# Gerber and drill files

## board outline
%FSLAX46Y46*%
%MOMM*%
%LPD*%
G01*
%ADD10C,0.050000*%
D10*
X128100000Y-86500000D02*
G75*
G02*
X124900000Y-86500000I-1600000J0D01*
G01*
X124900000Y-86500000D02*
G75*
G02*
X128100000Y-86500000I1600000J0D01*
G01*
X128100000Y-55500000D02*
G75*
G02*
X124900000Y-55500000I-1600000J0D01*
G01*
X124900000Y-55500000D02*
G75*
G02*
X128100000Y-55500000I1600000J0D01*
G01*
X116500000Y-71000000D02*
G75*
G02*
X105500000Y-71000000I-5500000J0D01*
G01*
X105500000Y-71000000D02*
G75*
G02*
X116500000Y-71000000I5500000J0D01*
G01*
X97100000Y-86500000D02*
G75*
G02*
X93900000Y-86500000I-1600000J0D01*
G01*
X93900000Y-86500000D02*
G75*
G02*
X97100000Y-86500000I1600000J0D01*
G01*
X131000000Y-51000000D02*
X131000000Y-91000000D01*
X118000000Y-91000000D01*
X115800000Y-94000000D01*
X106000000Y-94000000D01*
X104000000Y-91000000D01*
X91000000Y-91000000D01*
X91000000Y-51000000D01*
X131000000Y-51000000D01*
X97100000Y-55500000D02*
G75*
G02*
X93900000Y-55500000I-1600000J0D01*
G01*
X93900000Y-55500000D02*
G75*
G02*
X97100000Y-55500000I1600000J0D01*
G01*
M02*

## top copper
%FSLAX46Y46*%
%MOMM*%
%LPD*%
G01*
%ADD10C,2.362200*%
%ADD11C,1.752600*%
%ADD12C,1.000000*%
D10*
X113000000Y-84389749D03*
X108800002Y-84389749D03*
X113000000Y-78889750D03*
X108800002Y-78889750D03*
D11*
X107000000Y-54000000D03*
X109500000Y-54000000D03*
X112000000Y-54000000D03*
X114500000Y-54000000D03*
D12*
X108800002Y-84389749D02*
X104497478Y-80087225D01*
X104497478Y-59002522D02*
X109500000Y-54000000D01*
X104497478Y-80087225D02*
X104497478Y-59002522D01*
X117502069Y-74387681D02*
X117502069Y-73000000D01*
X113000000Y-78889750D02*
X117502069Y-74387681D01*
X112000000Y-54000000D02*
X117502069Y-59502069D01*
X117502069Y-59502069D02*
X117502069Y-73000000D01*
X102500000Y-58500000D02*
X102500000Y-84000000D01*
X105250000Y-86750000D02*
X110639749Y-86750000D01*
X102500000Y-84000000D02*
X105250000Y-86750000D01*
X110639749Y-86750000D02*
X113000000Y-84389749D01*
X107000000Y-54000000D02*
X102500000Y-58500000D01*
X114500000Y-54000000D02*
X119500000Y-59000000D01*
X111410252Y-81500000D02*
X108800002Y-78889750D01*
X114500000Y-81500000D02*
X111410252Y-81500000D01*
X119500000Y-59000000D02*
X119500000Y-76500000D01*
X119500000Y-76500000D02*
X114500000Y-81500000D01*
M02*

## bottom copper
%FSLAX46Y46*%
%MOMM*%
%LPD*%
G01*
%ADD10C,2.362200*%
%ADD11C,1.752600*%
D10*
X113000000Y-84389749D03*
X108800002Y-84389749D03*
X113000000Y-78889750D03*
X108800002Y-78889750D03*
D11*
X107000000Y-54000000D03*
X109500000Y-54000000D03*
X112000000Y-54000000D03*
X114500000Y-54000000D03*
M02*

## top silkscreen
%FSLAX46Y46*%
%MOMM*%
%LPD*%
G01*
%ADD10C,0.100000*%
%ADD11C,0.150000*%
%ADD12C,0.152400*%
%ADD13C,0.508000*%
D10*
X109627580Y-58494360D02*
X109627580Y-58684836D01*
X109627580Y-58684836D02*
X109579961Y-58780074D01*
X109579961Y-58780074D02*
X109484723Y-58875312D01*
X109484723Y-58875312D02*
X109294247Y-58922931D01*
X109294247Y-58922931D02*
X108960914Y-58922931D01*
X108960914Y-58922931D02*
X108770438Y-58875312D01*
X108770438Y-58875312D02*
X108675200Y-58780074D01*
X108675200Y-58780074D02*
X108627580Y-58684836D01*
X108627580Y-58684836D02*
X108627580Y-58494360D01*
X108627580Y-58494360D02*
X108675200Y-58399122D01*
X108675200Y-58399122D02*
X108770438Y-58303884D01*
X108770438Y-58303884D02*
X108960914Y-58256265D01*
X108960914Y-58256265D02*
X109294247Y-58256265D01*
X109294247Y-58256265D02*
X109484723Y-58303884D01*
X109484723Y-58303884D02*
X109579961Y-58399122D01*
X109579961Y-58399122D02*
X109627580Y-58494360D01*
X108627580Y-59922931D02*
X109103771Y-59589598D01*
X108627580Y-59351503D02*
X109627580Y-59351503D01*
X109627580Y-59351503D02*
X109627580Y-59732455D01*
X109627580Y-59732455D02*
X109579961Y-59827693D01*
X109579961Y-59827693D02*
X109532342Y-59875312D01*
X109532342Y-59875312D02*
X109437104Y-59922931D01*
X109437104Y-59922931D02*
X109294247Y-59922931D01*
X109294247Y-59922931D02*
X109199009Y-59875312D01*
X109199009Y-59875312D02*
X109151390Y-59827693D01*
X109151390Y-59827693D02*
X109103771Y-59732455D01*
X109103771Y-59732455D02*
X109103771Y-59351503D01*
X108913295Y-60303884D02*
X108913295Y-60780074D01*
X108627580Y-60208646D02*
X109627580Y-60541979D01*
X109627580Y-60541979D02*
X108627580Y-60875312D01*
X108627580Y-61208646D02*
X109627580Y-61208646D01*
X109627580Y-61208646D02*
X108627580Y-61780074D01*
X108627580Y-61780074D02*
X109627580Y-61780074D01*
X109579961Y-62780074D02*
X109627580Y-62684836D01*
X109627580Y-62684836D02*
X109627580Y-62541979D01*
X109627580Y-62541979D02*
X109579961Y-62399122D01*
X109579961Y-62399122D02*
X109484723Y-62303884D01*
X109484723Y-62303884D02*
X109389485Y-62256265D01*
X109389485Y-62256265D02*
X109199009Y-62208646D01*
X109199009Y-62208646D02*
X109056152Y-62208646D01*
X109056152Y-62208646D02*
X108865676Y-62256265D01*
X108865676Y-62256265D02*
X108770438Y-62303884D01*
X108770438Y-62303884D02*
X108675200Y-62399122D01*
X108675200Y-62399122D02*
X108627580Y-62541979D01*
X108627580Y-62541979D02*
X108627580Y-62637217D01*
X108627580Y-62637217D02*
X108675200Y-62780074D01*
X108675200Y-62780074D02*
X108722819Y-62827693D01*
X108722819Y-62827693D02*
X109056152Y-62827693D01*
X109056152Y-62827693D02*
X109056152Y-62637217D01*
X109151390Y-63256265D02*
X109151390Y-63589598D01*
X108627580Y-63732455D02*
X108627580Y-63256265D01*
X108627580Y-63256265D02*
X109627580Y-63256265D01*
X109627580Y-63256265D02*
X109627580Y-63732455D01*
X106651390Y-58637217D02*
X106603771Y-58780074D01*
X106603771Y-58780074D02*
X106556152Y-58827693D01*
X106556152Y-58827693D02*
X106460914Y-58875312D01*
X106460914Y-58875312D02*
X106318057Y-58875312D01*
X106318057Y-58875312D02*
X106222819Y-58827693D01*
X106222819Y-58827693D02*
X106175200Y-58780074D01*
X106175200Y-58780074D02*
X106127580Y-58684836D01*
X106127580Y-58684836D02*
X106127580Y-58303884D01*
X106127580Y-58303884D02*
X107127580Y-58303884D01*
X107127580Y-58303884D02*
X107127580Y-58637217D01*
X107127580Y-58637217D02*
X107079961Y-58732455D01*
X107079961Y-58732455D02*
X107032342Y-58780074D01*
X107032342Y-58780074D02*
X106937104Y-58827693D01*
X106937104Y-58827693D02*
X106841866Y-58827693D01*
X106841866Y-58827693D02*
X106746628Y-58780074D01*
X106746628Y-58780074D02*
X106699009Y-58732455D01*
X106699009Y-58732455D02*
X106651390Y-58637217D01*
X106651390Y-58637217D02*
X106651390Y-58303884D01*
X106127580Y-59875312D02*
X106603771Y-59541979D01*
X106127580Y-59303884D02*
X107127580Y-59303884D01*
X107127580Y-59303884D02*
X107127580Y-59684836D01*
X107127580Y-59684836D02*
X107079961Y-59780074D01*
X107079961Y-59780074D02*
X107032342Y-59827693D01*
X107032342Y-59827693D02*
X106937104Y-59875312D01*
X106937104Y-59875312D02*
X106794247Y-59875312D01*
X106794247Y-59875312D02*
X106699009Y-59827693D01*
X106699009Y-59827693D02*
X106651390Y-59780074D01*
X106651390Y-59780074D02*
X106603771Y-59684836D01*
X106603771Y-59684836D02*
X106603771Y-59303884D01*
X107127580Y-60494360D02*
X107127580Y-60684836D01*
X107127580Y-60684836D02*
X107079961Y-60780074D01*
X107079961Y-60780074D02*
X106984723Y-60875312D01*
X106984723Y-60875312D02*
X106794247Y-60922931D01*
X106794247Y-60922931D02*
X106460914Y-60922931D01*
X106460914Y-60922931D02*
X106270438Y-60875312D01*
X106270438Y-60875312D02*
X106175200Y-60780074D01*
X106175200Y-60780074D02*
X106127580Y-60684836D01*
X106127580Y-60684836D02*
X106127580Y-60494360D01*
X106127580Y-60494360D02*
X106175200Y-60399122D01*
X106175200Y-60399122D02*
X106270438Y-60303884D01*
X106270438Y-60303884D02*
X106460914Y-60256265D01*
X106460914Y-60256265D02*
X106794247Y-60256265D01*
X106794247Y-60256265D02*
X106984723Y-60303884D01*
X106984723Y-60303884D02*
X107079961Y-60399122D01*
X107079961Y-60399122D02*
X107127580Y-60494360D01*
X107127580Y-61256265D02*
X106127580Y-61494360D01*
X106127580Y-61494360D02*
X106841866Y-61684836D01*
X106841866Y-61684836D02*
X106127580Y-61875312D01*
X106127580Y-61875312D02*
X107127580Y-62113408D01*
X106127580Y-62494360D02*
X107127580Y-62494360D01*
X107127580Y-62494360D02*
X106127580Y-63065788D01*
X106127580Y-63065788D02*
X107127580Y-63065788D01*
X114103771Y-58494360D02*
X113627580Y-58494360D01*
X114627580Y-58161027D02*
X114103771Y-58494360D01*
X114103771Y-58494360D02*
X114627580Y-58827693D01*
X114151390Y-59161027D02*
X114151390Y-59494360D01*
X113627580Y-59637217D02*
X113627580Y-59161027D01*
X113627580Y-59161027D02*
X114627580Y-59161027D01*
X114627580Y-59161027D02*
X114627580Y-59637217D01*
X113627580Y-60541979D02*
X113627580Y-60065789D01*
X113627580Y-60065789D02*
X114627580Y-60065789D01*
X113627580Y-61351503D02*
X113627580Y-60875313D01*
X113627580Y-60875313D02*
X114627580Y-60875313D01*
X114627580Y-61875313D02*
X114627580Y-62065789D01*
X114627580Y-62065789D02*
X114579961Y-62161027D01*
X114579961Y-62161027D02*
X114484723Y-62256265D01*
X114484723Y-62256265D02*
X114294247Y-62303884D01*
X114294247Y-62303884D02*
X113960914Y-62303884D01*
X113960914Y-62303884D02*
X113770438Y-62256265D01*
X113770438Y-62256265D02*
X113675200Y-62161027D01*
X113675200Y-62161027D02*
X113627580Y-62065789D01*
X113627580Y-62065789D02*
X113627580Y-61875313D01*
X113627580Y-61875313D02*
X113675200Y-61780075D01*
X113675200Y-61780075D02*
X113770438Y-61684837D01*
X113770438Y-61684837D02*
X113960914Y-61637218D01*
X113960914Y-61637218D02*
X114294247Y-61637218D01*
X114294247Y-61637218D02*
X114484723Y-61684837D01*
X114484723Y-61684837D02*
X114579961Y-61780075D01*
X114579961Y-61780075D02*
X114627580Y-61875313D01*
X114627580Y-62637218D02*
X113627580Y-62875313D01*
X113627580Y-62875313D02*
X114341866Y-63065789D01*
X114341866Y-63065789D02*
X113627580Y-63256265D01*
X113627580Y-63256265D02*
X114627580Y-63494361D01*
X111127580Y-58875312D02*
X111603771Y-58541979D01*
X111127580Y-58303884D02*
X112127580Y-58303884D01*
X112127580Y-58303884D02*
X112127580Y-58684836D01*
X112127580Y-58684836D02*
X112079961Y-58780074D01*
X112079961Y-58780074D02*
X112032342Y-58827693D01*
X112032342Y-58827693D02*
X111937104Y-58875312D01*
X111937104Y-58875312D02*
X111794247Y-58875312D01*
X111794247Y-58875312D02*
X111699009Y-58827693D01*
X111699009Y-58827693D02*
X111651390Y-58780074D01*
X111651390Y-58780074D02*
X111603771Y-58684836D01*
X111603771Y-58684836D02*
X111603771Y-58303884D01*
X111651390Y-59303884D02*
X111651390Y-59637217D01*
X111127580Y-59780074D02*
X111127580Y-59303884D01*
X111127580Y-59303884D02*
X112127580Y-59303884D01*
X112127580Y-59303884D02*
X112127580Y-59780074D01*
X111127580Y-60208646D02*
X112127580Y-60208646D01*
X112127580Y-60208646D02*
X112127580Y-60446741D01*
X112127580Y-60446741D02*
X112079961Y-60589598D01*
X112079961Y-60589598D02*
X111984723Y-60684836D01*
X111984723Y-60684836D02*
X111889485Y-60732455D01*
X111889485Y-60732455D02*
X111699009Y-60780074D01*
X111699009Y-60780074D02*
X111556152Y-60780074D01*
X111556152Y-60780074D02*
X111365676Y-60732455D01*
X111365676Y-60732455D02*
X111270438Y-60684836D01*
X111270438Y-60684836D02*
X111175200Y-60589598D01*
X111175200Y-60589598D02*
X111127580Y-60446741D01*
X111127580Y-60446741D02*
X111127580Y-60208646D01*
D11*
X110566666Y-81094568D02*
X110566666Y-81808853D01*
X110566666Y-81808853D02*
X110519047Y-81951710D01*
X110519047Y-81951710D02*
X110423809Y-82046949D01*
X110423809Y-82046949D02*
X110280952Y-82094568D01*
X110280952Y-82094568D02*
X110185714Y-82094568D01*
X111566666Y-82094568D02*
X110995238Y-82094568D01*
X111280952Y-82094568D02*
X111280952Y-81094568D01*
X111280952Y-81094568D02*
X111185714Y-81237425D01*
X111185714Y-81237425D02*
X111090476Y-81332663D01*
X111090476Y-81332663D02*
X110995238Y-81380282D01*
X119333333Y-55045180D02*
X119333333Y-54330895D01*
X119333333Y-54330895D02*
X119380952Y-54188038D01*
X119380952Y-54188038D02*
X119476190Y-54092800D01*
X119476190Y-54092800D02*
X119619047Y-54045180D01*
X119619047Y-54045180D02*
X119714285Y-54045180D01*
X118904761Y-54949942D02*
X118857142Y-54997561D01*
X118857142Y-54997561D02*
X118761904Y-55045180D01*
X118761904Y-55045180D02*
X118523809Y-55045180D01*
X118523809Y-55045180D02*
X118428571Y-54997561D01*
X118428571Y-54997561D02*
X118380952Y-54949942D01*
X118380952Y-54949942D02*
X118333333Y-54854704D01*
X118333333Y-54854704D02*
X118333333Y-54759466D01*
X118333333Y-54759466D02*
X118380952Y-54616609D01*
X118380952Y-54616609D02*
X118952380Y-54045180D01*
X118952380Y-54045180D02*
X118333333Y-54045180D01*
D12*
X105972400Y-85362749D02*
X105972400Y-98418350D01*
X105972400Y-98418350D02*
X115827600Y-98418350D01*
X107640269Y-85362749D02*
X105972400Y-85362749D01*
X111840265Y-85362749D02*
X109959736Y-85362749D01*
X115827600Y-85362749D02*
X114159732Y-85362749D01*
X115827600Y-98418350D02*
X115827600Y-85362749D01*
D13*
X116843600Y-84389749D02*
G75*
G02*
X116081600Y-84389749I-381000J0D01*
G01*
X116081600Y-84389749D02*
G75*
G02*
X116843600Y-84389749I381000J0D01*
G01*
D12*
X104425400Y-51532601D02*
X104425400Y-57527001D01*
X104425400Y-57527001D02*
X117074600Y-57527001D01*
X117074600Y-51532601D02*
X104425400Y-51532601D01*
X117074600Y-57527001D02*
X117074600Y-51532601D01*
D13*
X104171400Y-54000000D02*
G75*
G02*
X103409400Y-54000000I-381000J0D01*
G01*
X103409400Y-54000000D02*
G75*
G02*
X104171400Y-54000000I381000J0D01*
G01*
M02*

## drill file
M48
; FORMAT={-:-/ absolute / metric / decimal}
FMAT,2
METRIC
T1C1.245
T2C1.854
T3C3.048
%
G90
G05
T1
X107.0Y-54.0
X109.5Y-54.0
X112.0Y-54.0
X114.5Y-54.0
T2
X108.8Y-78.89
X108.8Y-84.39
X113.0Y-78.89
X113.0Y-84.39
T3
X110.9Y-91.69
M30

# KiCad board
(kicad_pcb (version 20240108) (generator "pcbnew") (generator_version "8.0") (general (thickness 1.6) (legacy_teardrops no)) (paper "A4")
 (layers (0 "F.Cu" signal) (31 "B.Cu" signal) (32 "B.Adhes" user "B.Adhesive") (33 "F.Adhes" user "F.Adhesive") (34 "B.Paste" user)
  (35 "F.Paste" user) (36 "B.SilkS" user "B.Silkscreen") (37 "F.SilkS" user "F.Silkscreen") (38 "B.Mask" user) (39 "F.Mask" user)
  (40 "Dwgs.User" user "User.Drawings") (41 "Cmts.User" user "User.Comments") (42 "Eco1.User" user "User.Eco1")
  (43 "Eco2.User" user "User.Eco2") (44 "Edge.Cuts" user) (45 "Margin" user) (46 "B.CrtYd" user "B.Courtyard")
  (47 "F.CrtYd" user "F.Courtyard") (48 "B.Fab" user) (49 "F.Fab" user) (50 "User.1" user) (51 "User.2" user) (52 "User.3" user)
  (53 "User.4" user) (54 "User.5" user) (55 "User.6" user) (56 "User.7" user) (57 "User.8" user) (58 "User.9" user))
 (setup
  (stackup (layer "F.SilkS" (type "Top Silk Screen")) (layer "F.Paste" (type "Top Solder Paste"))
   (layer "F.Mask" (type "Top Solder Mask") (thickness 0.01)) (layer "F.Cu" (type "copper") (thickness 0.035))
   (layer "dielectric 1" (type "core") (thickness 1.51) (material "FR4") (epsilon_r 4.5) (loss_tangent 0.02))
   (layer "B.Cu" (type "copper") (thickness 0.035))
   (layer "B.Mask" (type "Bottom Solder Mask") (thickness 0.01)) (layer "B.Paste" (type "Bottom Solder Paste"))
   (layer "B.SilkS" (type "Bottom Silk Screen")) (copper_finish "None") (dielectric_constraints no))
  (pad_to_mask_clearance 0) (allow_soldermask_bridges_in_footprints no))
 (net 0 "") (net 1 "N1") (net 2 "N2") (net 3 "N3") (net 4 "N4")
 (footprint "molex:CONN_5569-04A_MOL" (layer "F.Cu") (at 113 84.389749)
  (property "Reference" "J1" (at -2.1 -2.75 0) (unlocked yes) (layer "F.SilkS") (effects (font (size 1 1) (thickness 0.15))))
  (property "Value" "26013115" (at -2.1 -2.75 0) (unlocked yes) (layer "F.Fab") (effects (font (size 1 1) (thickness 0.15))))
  (fp_line (start -7.0276 0.973) (end -7.0276 14.028601) (stroke (width 0.1524) (type solid)) (layer "F.SilkS"))
  (fp_line (start -7.0276 14.028601) (end 2.8276 14.028601) (stroke (width 0.1524) (type solid)) (layer "F.SilkS"))
  (fp_line (start -5.359731 0.973) (end -7.0276 0.973) (stroke (width 0.1524) (type solid)) (layer "F.SilkS"))
  (fp_line (start -1.159735 0.973) (end -3.040264 0.973) (stroke (width 0.1524) (type solid)) (layer "F.SilkS"))
  (fp_line (start 2.8276 0.973) (end 1.159732 0.973) (stroke (width 0.1524) (type solid)) (layer "F.SilkS"))
  (fp_line (start 2.8276 14.028601) (end 2.8276 0.973) (stroke (width 0.1524) (type solid)) (layer "F.SilkS"))
  (fp_circle (center 3.4626 0) (end 3.8436 0) (stroke (width 0.508) (type solid)) (fill none) (layer "F.SilkS"))
  (pad "" np_thru_hole circle (at -2.1 7.300001) (size 3.048 3.048) (drill 3.048) (layers))
  (pad "1" thru_hole circle (at 0 0) (size 2.3622 2.3622) (drill 1.8542) (layers "*.Cu" "*.Mask") (remove_unused_layers no) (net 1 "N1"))
  (pad "2" thru_hole circle (at -4.199998 0) (size 2.3622 2.3622) (drill 1.8542) (layers "*.Cu" "*.Mask") (remove_unused_layers no)
   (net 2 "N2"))
  (pad "3" thru_hole circle (at 0 -5.499999) (size 2.3622 2.3622) (drill 1.8542) (layers "*.Cu" "*.Mask") (remove_unused_layers no)
   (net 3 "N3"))
  (pad "4" thru_hole circle (at -4.199998 -5.499999) (size 2.3622 2.3622) (drill 1.8542) (layers "*.Cu" "*.Mask") (remove_unused_layers no)
   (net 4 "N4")))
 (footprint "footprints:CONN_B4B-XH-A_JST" (layer "F.Cu") (at 107 54 180)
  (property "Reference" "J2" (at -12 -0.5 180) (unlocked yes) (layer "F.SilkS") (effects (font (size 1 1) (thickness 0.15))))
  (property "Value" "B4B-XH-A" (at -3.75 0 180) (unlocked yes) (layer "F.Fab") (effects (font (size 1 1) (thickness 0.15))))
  (fp_line (start 2.5746 2.467399) (end 2.5746 -3.527001) (stroke (width 0.1524) (type solid)) (layer "F.SilkS"))
  (fp_line (start 2.5746 -3.527001) (end -10.0746 -3.527001) (stroke (width 0.1524) (type solid)) (layer "F.SilkS"))
  (fp_line (start -10.0746 2.467399) (end 2.5746 2.467399) (stroke (width 0.1524) (type solid)) (layer "F.SilkS"))
  (fp_line (start -10.0746 -3.527001) (end -10.0746 2.467399) (stroke (width 0.1524) (type solid)) (layer "F.SilkS"))
  (fp_circle (center 3.2096 0) (end 3.5906 0) (stroke (width 0.508) (type solid)) (fill none) (layer "F.SilkS"))
  (pad "1" thru_hole circle (at 0 0 180) (size 1.7526 1.7526) (drill 1.2446) (layers "*.Cu" "*.Mask") (remove_unused_layers no) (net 1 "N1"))
  (pad "2" thru_hole circle (at -2.5 0 180) (size 1.7526 1.7526) (drill 1.2446) (layers "*.Cu" "*.Mask") (remove_unused_layers no)
   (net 2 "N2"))
  (pad "3" thru_hole circle (at -5 0 180) (size 1.7526 1.7526) (drill 1.2446) (layers "*.Cu" "*.Mask") (remove_unused_layers no)
   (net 3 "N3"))
  (pad "4" thru_hole circle (at -7.5 0 180) (size 1.7526 1.7526) (drill 1.2446) (layers "*.Cu" "*.Mask") (remove_unused_layers no)
   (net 4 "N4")))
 (gr_circle (center 126.5 86.5) (end 128.1 86.5) (stroke (width 0.05) (type default)) (fill none) (layer "Edge.Cuts"))
 (gr_circle (center 126.5 55.5) (end 128.1 55.5) (stroke (width 0.05) (type default)) (fill none) (layer "Edge.Cuts"))
 (gr_circle (center 111 71) (end 116.5 71) (stroke (width 0.05) (type default)) (fill none) (layer "Edge.Cuts"))
 (gr_circle (center 95.5 86.5) (end 97.1 86.5) (stroke (width 0.05) (type default)) (fill none) (layer "Edge.Cuts"))
 (gr_poly
  (pts (xy 131 51) (xy 131 91) (xy 118 91) (xy 115.8 94) (xy 106 94) (xy 104 91) (xy 91 91) (xy 91 51)) (stroke (width 0.05) (type solid))
  (fill none) (layer "Edge.Cuts"))
 (gr_circle (center 95.5 55.5) (end 97.1 55.5) (stroke (width 0.05) (type default)) (fill none) (layer "Edge.Cuts"))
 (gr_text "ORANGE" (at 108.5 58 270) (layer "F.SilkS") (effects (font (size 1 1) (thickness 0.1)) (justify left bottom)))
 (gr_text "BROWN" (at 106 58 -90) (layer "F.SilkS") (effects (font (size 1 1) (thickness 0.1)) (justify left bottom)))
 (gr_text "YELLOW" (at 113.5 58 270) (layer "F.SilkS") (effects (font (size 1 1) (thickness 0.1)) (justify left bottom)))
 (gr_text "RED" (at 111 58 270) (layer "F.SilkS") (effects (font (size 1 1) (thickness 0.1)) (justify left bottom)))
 (segment (start 108.800002 84.389749) (end 104.497478 80.087225) (width 1) (layer "F.Cu") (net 2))
 (segment (start 104.497478 59.002522) (end 109.5 54) (width 1) (layer "F.Cu") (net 2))
 (segment (start 104.497478 80.087225) (end 104.497478 59.002522) (width 1) (layer "F.Cu") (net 2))
 (segment (start 117.502069 74.387681) (end 117.502069 73) (width 1) (layer "F.Cu") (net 3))
 (segment (start 113 78.88975) (end 117.502069 74.387681) (width 1) (layer "F.Cu") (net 3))
 (segment (start 112 54) (end 117.502069 59.502069) (width 1) (layer "F.Cu") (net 3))
 (segment (start 117.502069 59.502069) (end 117.502069 73) (width 1) (layer "F.Cu") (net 3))
 (segment (start 102.5 58.5) (end 102.5 84) (width 1) (layer "F.Cu") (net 1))
 (segment (start 105.25 86.75) (end 110.639749 86.75) (width 1) (layer "F.Cu") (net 1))
 (segment (start 102.5 84) (end 105.25 86.75) (width 1) (layer "F.Cu") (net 1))
 (segment (start 110.639749 86.75) (end 113 84.389749) (width 1) (layer "F.Cu") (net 1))
 (segment (start 107 54) (end 102.5 58.5) (width 1) (layer "F.Cu") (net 1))
 (segment (start 114.5 54) (end 119.5 59) (width 1) (layer "F.Cu") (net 4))
 (segment (start 111.410252 81.5) (end 108.800002 78.88975) (width 1) (layer "F.Cu") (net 4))
 (segment (start 114.5 81.5) (end 111.410252 81.5) (width 1) (layer "F.Cu") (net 4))
 (segment (start 119.5 59) (end 119.5 76.5) (width 1) (layer "F.Cu") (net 4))
 (segment (start 119.5 76.5) (end 114.5 81.5) (width 1) (layer "F.Cu") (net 4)))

